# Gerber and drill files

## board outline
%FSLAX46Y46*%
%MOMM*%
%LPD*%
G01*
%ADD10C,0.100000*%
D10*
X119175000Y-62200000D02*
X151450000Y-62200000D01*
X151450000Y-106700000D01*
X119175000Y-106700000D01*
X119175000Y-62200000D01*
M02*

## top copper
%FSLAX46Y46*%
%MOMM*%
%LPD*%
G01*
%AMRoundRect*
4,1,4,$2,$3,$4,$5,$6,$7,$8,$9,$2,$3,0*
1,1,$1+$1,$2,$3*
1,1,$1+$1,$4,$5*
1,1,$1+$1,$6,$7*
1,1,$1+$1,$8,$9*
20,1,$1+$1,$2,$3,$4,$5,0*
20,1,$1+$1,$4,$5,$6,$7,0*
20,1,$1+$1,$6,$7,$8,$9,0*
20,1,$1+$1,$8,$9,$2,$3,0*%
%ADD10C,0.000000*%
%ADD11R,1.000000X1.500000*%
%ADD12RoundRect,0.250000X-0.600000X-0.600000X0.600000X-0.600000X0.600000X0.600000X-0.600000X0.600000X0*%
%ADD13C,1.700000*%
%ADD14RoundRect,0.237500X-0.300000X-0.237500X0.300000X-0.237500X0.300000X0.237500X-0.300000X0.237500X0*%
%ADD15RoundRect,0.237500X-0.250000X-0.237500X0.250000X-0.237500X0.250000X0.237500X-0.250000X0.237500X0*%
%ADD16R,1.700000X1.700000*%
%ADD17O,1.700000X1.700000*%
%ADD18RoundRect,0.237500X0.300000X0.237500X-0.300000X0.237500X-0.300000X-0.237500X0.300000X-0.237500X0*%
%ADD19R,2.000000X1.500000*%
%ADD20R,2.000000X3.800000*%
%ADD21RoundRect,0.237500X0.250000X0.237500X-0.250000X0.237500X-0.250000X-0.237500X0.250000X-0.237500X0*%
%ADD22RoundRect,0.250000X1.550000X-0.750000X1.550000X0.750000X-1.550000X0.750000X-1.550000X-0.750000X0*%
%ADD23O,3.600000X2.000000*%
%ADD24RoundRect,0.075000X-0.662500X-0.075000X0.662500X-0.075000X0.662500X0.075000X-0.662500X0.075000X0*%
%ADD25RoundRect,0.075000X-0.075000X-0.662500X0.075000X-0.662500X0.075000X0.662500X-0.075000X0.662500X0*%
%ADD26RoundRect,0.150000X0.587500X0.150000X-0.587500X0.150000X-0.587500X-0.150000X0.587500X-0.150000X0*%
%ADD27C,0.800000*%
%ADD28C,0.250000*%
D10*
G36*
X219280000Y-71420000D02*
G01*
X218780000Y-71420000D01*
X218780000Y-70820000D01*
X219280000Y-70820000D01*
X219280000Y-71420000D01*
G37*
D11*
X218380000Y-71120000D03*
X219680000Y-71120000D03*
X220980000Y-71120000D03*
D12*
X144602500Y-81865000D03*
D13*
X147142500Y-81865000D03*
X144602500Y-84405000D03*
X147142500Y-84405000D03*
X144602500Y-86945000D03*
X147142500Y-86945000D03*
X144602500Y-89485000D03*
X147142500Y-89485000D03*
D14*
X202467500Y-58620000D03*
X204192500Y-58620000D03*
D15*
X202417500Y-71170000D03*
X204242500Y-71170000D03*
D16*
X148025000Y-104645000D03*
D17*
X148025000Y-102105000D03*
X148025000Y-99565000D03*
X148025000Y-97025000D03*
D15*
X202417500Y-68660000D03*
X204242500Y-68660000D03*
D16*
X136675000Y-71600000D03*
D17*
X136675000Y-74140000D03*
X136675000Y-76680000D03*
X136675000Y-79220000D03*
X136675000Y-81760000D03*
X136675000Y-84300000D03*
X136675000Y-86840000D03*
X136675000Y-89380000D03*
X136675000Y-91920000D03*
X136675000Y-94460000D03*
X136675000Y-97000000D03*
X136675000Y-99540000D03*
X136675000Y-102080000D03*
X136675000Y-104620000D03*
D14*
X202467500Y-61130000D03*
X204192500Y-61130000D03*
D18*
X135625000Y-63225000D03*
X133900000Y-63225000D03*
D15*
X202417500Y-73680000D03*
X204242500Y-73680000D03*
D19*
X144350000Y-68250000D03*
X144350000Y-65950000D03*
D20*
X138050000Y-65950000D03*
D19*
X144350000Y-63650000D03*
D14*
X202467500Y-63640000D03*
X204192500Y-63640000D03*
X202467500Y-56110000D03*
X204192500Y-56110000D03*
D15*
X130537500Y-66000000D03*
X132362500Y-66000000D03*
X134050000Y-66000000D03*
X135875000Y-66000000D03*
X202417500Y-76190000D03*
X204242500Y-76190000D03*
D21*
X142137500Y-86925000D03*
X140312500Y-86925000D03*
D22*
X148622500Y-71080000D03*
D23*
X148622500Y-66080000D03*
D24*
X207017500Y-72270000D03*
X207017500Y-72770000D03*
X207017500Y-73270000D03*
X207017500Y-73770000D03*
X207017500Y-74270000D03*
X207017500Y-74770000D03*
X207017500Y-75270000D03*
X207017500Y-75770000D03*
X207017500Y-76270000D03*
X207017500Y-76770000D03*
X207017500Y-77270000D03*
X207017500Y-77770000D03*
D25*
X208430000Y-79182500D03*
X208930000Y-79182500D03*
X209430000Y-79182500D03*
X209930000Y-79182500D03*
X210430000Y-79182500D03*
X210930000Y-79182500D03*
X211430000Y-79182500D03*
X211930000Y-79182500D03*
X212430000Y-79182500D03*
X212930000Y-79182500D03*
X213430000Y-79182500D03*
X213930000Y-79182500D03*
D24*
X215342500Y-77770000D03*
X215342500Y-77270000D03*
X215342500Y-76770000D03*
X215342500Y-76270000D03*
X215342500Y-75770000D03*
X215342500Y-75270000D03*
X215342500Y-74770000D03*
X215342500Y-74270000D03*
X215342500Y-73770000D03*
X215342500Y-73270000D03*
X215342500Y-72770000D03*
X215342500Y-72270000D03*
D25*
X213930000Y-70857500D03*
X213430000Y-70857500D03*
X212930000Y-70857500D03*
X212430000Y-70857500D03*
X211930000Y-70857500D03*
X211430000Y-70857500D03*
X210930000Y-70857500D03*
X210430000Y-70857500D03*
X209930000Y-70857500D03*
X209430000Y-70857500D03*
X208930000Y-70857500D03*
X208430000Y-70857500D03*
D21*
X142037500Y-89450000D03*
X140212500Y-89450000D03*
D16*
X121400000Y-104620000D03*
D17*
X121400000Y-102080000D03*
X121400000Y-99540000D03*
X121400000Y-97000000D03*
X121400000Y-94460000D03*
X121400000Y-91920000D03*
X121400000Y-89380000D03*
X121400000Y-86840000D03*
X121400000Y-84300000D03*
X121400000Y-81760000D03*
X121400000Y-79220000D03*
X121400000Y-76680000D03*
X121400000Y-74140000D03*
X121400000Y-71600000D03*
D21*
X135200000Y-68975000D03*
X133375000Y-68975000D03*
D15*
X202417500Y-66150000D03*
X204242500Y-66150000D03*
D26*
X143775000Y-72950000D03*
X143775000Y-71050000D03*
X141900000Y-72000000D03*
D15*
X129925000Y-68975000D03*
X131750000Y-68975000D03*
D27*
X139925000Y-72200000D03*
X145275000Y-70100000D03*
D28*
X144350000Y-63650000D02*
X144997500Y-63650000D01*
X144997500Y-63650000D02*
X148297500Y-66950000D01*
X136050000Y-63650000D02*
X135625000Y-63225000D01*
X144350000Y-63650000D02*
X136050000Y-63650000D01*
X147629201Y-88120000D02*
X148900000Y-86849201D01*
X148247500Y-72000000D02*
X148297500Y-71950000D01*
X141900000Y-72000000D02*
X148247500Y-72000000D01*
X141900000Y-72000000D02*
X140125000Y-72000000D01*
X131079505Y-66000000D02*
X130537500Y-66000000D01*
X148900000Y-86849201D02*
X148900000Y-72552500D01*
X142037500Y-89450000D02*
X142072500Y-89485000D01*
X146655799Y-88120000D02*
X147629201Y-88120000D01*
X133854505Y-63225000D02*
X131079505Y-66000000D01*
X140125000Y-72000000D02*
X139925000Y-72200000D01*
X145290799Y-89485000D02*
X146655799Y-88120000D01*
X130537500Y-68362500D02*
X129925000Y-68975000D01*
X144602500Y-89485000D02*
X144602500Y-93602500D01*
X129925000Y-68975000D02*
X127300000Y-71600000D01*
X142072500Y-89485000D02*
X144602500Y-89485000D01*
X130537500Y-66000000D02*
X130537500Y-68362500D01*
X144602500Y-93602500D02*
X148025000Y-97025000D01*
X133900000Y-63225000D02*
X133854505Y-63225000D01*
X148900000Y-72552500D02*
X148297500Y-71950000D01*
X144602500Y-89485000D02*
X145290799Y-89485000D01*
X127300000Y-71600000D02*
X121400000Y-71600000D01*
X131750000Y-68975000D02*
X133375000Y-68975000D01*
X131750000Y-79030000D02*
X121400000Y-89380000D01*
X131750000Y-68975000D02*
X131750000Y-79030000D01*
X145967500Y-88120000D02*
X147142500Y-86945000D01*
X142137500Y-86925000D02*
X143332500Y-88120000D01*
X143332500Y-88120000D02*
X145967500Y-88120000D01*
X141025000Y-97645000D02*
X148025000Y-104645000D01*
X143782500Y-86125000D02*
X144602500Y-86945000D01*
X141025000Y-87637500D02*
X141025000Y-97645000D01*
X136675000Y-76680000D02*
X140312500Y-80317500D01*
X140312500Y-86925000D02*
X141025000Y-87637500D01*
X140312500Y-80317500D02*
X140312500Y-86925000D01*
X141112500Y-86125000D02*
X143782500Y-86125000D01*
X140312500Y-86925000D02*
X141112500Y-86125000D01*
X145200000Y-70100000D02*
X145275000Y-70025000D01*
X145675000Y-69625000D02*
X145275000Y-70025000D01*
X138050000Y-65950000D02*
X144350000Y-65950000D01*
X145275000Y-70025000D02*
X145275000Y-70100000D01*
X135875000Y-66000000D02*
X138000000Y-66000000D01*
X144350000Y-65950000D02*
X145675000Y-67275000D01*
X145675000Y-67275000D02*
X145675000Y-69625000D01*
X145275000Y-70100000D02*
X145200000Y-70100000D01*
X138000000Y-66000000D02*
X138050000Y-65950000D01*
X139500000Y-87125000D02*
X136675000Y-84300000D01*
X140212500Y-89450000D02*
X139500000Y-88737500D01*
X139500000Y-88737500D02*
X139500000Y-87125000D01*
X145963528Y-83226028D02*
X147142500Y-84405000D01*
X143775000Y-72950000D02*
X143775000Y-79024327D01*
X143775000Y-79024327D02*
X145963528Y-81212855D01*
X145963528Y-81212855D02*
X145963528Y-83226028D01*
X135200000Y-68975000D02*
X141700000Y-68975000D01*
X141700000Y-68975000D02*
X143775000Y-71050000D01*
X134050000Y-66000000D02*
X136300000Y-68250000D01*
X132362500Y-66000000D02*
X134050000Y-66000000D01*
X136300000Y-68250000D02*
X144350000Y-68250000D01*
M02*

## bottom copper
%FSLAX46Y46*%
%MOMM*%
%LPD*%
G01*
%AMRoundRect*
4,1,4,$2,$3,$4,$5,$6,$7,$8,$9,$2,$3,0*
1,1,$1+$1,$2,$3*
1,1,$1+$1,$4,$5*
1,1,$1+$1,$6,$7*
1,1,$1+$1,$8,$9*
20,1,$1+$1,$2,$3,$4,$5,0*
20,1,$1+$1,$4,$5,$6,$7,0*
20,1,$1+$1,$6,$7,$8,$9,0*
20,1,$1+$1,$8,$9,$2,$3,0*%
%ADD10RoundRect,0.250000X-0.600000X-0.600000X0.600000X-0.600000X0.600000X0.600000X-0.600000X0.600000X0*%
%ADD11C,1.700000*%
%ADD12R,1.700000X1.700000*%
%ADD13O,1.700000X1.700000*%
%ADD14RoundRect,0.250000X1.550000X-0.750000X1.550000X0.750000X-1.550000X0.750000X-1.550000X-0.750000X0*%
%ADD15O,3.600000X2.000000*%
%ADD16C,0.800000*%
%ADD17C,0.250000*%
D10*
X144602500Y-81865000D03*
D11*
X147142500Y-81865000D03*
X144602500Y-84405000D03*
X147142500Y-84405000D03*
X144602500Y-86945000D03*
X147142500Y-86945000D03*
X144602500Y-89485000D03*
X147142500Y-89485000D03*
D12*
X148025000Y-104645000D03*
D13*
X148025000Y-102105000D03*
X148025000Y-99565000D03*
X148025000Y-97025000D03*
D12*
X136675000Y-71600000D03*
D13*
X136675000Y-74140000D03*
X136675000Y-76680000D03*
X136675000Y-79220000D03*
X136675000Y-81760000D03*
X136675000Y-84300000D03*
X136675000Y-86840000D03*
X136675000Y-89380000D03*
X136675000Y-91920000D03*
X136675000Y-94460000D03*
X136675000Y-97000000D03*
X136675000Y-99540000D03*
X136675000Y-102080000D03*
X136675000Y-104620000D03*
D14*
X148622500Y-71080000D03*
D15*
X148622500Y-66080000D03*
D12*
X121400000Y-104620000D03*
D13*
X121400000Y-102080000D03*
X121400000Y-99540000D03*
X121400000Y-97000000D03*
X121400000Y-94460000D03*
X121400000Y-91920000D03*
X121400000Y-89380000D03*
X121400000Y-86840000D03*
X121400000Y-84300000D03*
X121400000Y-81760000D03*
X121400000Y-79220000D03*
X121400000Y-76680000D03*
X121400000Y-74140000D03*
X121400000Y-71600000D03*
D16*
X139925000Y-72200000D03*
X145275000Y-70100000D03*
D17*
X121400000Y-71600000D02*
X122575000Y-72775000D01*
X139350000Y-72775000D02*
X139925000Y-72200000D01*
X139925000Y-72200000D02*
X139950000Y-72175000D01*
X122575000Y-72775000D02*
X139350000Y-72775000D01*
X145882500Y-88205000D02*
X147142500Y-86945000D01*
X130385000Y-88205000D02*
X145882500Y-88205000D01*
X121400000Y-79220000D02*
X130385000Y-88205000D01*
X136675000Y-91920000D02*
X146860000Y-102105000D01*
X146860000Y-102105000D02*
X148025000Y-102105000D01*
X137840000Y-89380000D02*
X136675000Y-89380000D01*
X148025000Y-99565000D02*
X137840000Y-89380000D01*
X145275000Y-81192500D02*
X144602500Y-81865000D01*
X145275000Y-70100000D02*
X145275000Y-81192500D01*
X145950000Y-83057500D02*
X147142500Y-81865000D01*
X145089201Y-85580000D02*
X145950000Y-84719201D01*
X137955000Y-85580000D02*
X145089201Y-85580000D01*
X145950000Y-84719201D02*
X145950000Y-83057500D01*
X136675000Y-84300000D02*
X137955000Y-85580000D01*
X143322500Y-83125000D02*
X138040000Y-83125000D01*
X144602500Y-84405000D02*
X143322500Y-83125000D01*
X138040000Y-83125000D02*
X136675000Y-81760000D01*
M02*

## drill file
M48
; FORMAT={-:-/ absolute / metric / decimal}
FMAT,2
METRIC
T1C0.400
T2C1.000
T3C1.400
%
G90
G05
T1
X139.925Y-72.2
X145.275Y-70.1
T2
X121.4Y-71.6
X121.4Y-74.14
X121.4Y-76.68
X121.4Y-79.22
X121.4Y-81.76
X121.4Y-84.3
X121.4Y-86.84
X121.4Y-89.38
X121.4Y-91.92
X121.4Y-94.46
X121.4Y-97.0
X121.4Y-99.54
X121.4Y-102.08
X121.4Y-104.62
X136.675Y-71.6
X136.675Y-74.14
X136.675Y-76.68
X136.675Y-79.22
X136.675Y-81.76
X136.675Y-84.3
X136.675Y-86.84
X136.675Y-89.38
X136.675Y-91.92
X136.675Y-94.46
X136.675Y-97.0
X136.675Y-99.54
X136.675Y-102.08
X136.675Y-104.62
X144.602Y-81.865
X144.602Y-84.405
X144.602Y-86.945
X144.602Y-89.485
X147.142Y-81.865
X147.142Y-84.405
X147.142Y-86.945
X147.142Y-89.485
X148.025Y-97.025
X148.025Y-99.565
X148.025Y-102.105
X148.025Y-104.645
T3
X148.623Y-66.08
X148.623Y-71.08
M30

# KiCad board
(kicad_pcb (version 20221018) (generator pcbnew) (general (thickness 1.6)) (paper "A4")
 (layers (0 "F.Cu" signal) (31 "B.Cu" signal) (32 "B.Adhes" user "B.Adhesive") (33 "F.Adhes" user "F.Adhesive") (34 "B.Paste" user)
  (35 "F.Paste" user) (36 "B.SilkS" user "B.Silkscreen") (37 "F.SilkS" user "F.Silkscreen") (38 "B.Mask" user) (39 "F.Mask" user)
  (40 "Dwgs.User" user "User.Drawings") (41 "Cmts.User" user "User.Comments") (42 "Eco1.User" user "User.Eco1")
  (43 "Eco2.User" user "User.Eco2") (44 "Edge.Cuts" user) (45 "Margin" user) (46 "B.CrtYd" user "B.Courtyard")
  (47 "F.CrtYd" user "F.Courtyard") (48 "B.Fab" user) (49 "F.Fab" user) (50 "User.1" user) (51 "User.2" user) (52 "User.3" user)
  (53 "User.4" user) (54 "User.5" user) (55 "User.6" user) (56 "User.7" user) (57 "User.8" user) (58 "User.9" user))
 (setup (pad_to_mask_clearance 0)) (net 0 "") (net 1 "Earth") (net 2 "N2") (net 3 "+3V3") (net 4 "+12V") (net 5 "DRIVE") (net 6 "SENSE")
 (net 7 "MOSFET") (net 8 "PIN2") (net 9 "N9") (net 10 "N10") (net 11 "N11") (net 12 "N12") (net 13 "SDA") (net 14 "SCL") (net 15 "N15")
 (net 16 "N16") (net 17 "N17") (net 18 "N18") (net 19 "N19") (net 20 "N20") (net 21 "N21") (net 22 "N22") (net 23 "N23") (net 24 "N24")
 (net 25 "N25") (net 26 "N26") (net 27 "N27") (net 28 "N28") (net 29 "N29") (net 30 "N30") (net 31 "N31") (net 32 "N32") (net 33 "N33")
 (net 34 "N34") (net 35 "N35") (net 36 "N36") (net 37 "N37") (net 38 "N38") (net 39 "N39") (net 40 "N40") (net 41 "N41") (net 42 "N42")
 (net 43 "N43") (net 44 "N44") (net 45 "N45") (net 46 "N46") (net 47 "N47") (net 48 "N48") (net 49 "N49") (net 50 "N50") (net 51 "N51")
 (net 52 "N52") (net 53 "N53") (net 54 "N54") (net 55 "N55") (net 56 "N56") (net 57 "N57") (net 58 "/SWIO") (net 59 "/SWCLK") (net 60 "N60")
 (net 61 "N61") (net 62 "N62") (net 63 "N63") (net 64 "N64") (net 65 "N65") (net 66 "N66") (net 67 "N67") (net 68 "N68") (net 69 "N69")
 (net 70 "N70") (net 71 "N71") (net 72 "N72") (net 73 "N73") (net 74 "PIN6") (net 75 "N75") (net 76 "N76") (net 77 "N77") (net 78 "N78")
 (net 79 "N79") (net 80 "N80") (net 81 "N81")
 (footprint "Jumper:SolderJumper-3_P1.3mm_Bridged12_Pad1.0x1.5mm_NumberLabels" (layer "F.Cu") (at 219.68 71.12)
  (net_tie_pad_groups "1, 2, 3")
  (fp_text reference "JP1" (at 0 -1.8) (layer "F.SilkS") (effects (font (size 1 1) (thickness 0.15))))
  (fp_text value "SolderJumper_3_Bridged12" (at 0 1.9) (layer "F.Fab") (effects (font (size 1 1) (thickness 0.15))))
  (fp_poly (pts (xy -0.9 -0.3) (xy -0.4 -0.3) (xy -0.4 0.3) (xy -0.9 0.3)) (stroke (width 0) (type solid)) (fill solid) (layer "F.Cu"))
  (pad "1" smd rect (at -1.3 0) (size 1 1.5) (layers "F.Cu" "F.Mask") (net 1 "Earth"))
  (pad "2" smd rect (at 0 0) (size 1 1.5) (layers "F.Cu" "F.Mask") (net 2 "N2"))
  (pad "3" smd rect (at 1.3 0) (size 1 1.5) (layers "F.Cu" "F.Mask") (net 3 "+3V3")))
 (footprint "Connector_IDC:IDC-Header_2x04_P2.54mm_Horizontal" (layer "F.Cu") (at 144.6025 81.865)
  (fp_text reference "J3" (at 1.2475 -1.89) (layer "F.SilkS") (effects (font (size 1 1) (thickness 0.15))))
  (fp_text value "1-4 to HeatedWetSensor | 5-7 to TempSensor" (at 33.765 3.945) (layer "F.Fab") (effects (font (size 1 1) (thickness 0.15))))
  (pad "1" thru_hole roundrect (at 0 0) (size 1.7 1.7) (drill 1) (layers "*.Cu" "*.Mask") (roundrect_rratio 0.147059) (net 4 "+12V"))
  (pad "2" thru_hole circle (at 2.54 0) (size 1.7 1.7) (drill 1) (layers "*.Cu" "*.Mask") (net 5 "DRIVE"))
  (pad "3" thru_hole circle (at 0 2.54) (size 1.7 1.7) (drill 1) (layers "*.Cu" "*.Mask") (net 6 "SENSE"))
  (pad "4" thru_hole circle (at 2.54 2.54) (size 1.7 1.7) (drill 1) (layers "*.Cu" "*.Mask") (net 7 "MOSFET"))
  (pad "5" thru_hole circle (at 0 5.08) (size 1.7 1.7) (drill 1) (layers "*.Cu" "*.Mask") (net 3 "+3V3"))
  (pad "6" thru_hole circle (at 2.54 5.08) (size 1.7 1.7) (drill 1) (layers "*.Cu" "*.Mask") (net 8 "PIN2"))
  (pad "7" thru_hole circle (at 0 7.62) (size 1.7 1.7) (drill 1) (layers "*.Cu" "*.Mask") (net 1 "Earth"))
  (pad "8" thru_hole circle (at 2.54 7.62) (size 1.7 1.7) (drill 1) (layers "*.Cu" "*.Mask") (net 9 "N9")))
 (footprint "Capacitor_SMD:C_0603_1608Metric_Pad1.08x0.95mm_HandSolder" (layer "F.Cu") (at 203.33 58.62)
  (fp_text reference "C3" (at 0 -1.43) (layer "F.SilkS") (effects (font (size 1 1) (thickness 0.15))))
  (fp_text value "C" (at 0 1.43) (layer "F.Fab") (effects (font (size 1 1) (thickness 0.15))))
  (pad "1" smd roundrect (at -0.8625 0) (size 1.075 0.95) (layers "F.Cu" "F.Paste" "F.Mask") (roundrect_rratio 0.25) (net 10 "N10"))
  (pad "2" smd roundrect (at 0.8625 0) (size 1.075 0.95) (layers "F.Cu" "F.Paste" "F.Mask") (roundrect_rratio 0.25) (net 1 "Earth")))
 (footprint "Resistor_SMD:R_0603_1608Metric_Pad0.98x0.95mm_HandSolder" (layer "F.Cu") (at 203.33 71.17)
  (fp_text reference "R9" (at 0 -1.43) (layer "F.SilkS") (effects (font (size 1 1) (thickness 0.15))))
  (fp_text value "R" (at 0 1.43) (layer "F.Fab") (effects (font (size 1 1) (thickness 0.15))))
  (pad "1" smd roundrect (at -0.9125 0) (size 0.975 0.95) (layers "F.Cu" "F.Paste" "F.Mask") (roundrect_rratio 0.25) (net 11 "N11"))
  (pad "2" smd roundrect (at 0.9125 0) (size 0.975 0.95) (layers "F.Cu" "F.Paste" "F.Mask") (roundrect_rratio 0.25) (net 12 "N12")))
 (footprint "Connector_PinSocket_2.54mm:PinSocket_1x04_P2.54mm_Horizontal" (layer "F.Cu") (at 148.025 104.645 180)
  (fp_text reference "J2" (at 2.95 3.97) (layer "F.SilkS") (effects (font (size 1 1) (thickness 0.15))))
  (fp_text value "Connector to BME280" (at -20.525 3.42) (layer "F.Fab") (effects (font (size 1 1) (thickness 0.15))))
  (pad "1" thru_hole rect (at 0 0 180) (size 1.7 1.7) (drill 1) (layers "*.Cu" "*.Mask") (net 3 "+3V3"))
  (pad "2" thru_hole oval (at 0 2.54 180) (size 1.7 1.7) (drill 1) (layers "*.Cu" "*.Mask") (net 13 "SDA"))
  (pad "3" thru_hole oval (at 0 5.08 180) (size 1.7 1.7) (drill 1) (layers "*.Cu" "*.Mask") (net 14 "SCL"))
  (pad "4" thru_hole oval (at 0 7.62 180) (size 1.7 1.7) (drill 1) (layers "*.Cu" "*.Mask") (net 1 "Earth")))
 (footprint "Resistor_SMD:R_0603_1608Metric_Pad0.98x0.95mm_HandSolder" (layer "F.Cu") (at 203.33 68.66)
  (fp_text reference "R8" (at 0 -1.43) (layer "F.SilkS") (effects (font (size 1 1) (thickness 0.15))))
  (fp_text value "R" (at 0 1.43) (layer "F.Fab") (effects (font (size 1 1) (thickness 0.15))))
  (pad "1" smd roundrect (at -0.9125 0) (size 0.975 0.95) (layers "F.Cu" "F.Paste" "F.Mask") (roundrect_rratio 0.25) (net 11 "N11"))
  (pad "2" smd roundrect (at 0.9125 0) (size 0.975 0.95) (layers "F.Cu" "F.Paste" "F.Mask") (roundrect_rratio 0.25) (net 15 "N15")))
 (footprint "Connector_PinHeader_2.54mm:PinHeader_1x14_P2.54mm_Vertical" (layer "F.Cu") (at 136.675 71.6)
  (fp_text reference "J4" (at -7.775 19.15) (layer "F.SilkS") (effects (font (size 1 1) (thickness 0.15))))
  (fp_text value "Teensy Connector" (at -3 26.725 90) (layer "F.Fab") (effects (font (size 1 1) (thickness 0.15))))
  (pad "1" thru_hole rect (at 0 0) (size 1.7 1.7) (drill 1) (layers "*.Cu" "*.Mask") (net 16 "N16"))
  (pad "2" thru_hole oval (at 0 2.54) (size 1.7 1.7) (drill 1) (layers "*.Cu" "*.Mask") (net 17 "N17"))
  (pad "3" thru_hole oval (at 0 5.08) (size 1.7 1.7) (drill 1) (layers "*.Cu" "*.Mask") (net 3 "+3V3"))
  (pad "4" thru_hole oval (at 0 7.62) (size 1.7 1.7) (drill 1) (layers "*.Cu" "*.Mask") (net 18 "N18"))
  (pad "5" thru_hole oval (at 0 10.16) (size 1.7 1.7) (drill 1) (layers "*.Cu" "*.Mask") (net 6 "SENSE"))
  (pad "6" thru_hole oval (at 0 12.7) (size 1.7 1.7) (drill 1) (layers "*.Cu" "*.Mask") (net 5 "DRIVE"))
  (pad "7" thru_hole oval (at 0 15.24) (size 1.7 1.7) (drill 1) (layers "*.Cu" "*.Mask") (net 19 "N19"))
  (pad "8" thru_hole oval (at 0 17.78) (size 1.7 1.7) (drill 1) (layers "*.Cu" "*.Mask") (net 14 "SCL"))
  (pad "9" thru_hole oval (at 0 20.32) (size 1.7 1.7) (drill 1) (layers "*.Cu" "*.Mask") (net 13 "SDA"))
  (pad "10" thru_hole oval (at 0 22.86) (size 1.7 1.7) (drill 1) (layers "*.Cu" "*.Mask") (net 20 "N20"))
  (pad "11" thru_hole oval (at 0 25.4) (size 1.7 1.7) (drill 1) (layers "*.Cu" "*.Mask") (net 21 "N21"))
  (pad "12" thru_hole oval (at 0 27.94) (size 1.7 1.7) (drill 1) (layers "*.Cu" "*.Mask") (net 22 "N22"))
  (pad "13" thru_hole oval (at 0 30.48) (size 1.7 1.7) (drill 1) (layers "*.Cu" "*.Mask") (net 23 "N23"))
  (pad "14" thru_hole oval (at 0 33.02) (size 1.7 1.7) (drill 1) (layers "*.Cu" "*.Mask") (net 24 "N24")))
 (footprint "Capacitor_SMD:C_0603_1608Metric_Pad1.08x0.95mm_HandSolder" (layer "F.Cu") (at 203.33 61.13)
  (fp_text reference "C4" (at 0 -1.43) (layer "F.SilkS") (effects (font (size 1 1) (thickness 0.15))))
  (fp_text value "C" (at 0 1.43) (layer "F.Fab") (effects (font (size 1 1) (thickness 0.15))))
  (pad "1" smd roundrect (at -0.8625 0) (size 1.075 0.95) (layers "F.Cu" "F.Paste" "F.Mask") (roundrect_rratio 0.25) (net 4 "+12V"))
  (pad "2" smd roundrect (at 0.8625 0) (size 1.075 0.95) (layers "F.Cu" "F.Paste" "F.Mask") (roundrect_rratio 0.25) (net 1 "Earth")))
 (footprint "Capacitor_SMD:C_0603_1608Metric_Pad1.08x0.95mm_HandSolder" (layer "F.Cu") (at 134.7625 63.225 180)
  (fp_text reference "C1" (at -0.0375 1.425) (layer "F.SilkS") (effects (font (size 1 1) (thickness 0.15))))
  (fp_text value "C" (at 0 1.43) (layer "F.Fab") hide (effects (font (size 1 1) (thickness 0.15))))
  (pad "1" smd roundrect (at -0.8625 0 180) (size 1.075 0.95) (layers "F.Cu" "F.Paste" "F.Mask") (roundrect_rratio 0.25) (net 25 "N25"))
  (pad "2" smd roundrect (at 0.8625 0 180) (size 1.075 0.95) (layers "F.Cu" "F.Paste" "F.Mask") (roundrect_rratio 0.25) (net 1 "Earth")))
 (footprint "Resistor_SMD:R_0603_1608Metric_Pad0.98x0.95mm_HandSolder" (layer "F.Cu") (at 203.33 73.68)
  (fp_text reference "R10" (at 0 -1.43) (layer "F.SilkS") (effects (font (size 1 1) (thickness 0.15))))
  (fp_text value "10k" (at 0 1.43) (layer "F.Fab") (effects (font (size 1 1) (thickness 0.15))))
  (pad "1" smd roundrect (at -0.9125 0) (size 0.975 0.95) (layers "F.Cu" "F.Paste" "F.Mask") (roundrect_rratio 0.25) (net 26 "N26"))
  (pad "2" smd roundrect (at 0.9125 0) (size 0.975 0.95) (layers "F.Cu" "F.Paste" "F.Mask") (roundrect_rratio 0.25) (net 3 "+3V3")))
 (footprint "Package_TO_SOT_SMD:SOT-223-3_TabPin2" (layer "F.Cu") (at 141.2 65.95 180)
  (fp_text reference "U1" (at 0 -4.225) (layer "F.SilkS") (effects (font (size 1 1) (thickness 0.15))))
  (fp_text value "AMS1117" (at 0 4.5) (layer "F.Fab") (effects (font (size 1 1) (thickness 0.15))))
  (pad "1" smd rect (at -3.15 -2.3 180) (size 2 1.5) (layers "F.Cu" "F.Paste" "F.Mask") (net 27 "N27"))
  (pad "2" smd rect (at -3.15 0 180) (size 2 1.5) (layers "F.Cu" "F.Paste" "F.Mask") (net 4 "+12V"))
  (pad "2" smd rect (at 3.15 0 180) (size 2 3.8) (layers "F.Cu" "F.Paste" "F.Mask") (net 4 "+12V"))
  (pad "3" smd rect (at -3.15 2.3 180) (size 2 1.5) (layers "F.Cu" "F.Paste" "F.Mask") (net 25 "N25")))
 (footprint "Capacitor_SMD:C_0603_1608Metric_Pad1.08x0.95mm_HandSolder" (layer "F.Cu") (at 203.33 63.64)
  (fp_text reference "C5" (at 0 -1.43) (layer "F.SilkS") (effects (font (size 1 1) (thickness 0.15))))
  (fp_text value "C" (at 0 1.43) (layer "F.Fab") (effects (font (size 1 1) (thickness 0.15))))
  (pad "1" smd roundrect (at -0.8625 0) (size 1.075 0.95) (layers "F.Cu" "F.Paste" "F.Mask") (roundrect_rratio 0.25) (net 26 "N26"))
  (pad "2" smd roundrect (at 0.8625 0) (size 1.075 0.95) (layers "F.Cu" "F.Paste" "F.Mask") (roundrect_rratio 0.25) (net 1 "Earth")))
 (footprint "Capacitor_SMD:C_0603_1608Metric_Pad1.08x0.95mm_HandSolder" (layer "F.Cu") (at 203.33 56.11)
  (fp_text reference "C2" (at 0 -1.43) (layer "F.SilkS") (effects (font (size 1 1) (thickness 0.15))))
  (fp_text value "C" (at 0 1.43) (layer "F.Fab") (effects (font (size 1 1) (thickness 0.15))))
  (pad "1" smd roundrect (at -0.8625 0) (size 1.075 0.95) (layers "F.Cu" "F.Paste" "F.Mask") (roundrect_rratio 0.25) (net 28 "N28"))
  (pad "2" smd roundrect (at 0.8625 0) (size 1.075 0.95) (layers "F.Cu" "F.Paste" "F.Mask") (roundrect_rratio 0.25) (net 1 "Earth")))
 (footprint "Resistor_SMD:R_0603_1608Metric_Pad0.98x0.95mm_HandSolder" (layer "F.Cu") (at 131.45 66)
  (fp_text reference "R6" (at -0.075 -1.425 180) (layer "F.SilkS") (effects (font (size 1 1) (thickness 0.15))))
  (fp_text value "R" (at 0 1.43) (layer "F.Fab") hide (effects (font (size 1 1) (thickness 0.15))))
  (pad "1" smd roundrect (at -0.9125 0) (size 0.975 0.95) (layers "F.Cu" "F.Paste" "F.Mask") (roundrect_rratio 0.25) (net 1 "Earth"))
  (pad "2" smd roundrect (at 0.9125 0) (size 0.975 0.95) (layers "F.Cu" "F.Paste" "F.Mask") (roundrect_rratio 0.25) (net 27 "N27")))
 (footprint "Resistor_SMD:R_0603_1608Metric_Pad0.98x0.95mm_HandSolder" (layer "F.Cu") (at 134.9625 66)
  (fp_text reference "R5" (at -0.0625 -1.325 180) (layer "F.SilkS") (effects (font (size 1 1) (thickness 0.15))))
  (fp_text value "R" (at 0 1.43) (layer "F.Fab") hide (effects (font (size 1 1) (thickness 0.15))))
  (pad "1" smd roundrect (at -0.9125 0) (size 0.975 0.95) (layers "F.Cu" "F.Paste" "F.Mask") (roundrect_rratio 0.25) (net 27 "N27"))
  (pad "2" smd roundrect (at 0.9125 0) (size 0.975 0.95) (layers "F.Cu" "F.Paste" "F.Mask") (roundrect_rratio 0.25) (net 4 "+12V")))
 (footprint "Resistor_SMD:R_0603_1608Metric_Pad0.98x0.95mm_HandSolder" (layer "F.Cu") (at 203.33 76.19)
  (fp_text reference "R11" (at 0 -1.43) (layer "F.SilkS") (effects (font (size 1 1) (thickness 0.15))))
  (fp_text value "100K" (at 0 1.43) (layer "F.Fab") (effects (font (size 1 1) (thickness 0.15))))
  (pad "1" smd roundrect (at -0.9125 0) (size 0.975 0.95) (layers "F.Cu" "F.Paste" "F.Mask") (roundrect_rratio 0.25) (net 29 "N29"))
  (pad "2" smd roundrect (at 0.9125 0) (size 0.975 0.95) (layers "F.Cu" "F.Paste" "F.Mask") (roundrect_rratio 0.25) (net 2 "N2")))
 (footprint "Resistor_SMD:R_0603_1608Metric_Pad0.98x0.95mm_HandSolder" (layer "F.Cu") (at 141.225 86.925 180)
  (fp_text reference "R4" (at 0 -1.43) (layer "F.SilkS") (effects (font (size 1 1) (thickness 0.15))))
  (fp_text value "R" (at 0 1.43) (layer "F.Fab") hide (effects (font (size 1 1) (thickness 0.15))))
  (pad "1" smd roundrect (at -0.9125 0 180) (size 0.975 0.95) (layers "F.Cu" "F.Paste" "F.Mask") (roundrect_rratio 0.25) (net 8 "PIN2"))
  (pad "2" smd roundrect (at 0.9125 0 180) (size 0.975 0.95) (layers "F.Cu" "F.Paste" "F.Mask") (roundrect_rratio 0.25) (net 3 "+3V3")))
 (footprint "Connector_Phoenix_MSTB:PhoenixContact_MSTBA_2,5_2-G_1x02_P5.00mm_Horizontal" (layer "F.Cu") (at 148.6225 71.08 90)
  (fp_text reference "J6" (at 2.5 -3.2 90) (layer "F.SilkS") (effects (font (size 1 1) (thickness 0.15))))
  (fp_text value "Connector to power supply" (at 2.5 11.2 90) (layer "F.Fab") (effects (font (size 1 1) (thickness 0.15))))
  (pad "1" thru_hole roundrect (at 0 0 90) (size 2 3.6) (drill 1.4) (layers "*.Cu" "*.Mask") (roundrect_rratio 0.125) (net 1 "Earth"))
  (pad "2" thru_hole oval (at 5 0 90) (size 2 3.6) (drill 1.4) (layers "*.Cu" "*.Mask") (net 10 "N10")))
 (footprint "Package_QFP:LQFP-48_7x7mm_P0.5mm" (layer "F.Cu") (at 211.18 75.02)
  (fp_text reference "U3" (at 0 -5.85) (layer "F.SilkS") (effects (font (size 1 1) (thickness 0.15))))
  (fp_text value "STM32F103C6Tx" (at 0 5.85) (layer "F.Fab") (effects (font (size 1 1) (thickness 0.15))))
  (pad "1" smd roundrect (at -4.1625 -2.75) (size 1.475 0.3) (layers "F.Cu" "F.Paste" "F.Mask") (roundrect_rratio 0.25) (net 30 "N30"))
  (pad "2" smd roundrect (at -4.1625 -2.25) (size 1.475 0.3) (layers "F.Cu" "F.Paste" "F.Mask") (roundrect_rratio 0.25) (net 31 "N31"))
  (pad "3" smd roundrect (at -4.1625 -1.75) (size 1.475 0.3) (layers "F.Cu" "F.Paste" "F.Mask") (roundrect_rratio 0.25) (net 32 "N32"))
  (pad "4" smd roundrect (at -4.1625 -1.25) (size 1.475 0.3) (layers "F.Cu" "F.Paste" "F.Mask") (roundrect_rratio 0.25) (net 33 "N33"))
  (pad "5" smd roundrect (at -4.1625 -0.75) (size 1.475 0.3) (layers "F.Cu" "F.Paste" "F.Mask") (roundrect_rratio 0.25) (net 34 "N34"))
  (pad "6" smd roundrect (at -4.1625 -0.25) (size 1.475 0.3) (layers "F.Cu" "F.Paste" "F.Mask") (roundrect_rratio 0.25) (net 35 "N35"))
  (pad "7" smd roundrect (at -4.1625 0.25) (size 1.475 0.3) (layers "F.Cu" "F.Paste" "F.Mask") (roundrect_rratio 0.25) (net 26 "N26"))
  (pad "8" smd roundrect (at -4.1625 0.75) (size 1.475 0.3) (layers "F.Cu" "F.Paste" "F.Mask") (roundrect_rratio 0.25) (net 1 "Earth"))
  (pad "9" smd roundrect (at -4.1625 1.25) (size 1.475 0.3) (layers "F.Cu" "F.Paste" "F.Mask") (roundrect_rratio 0.25) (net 3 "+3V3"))
  (pad "10" smd roundrect (at -4.1625 1.75) (size 1.475 0.3) (layers "F.Cu" "F.Paste" "F.Mask") (roundrect_rratio 0.25) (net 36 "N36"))
  (pad "11" smd roundrect (at -4.1625 2.25) (size 1.475 0.3) (layers "F.Cu" "F.Paste" "F.Mask") (roundrect_rratio 0.25) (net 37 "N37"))
  (pad "12" smd roundrect (at -4.1625 2.75) (size 1.475 0.3) (layers "F.Cu" "F.Paste" "F.Mask") (roundrect_rratio 0.25) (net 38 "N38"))
  (pad "13" smd roundrect (at -2.75 4.1625) (size 0.3 1.475) (layers "F.Cu" "F.Paste" "F.Mask") (roundrect_rratio 0.25) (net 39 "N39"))
  (pad "14" smd roundrect (at -2.25 4.1625) (size 0.3 1.475) (layers "F.Cu" "F.Paste" "F.Mask") (roundrect_rratio 0.25) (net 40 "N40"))
  (pad "15" smd roundrect (at -1.75 4.1625) (size 0.3 1.475) (layers "F.Cu" "F.Paste" "F.Mask") (roundrect_rratio 0.25) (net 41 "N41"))
  (pad "16" smd roundrect (at -1.25 4.1625) (size 0.3 1.475) (layers "F.Cu" "F.Paste" "F.Mask") (roundrect_rratio 0.25) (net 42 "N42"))
  (pad "17" smd roundrect (at -0.75 4.1625) (size 0.3 1.475) (layers "F.Cu" "F.Paste" "F.Mask") (roundrect_rratio 0.25) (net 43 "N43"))
  (pad "18" smd roundrect (at -0.25 4.1625) (size 0.3 1.475) (layers "F.Cu" "F.Paste" "F.Mask") (roundrect_rratio 0.25) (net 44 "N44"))
  (pad "19" smd roundrect (at 0.25 4.1625) (size 0.3 1.475) (layers "F.Cu" "F.Paste" "F.Mask") (roundrect_rratio 0.25) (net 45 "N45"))
  (pad "20" smd roundrect (at 0.75 4.1625) (size 0.3 1.475) (layers "F.Cu" "F.Paste" "F.Mask") (roundrect_rratio 0.25) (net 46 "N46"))
  (pad "21" smd roundrect (at 1.25 4.1625) (size 0.3 1.475) (layers "F.Cu" "F.Paste" "F.Mask") (roundrect_rratio 0.25) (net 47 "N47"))
  (pad "22" smd roundrect (at 1.75 4.1625) (size 0.3 1.475) (layers "F.Cu" "F.Paste" "F.Mask") (roundrect_rratio 0.25) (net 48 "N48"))
  (pad "23" smd roundrect (at 2.25 4.1625) (size 0.3 1.475) (layers "F.Cu" "F.Paste" "F.Mask") (roundrect_rratio 0.25) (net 1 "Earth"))
  (pad "24" smd roundrect (at 2.75 4.1625) (size 0.3 1.475) (layers "F.Cu" "F.Paste" "F.Mask") (roundrect_rratio 0.25) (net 3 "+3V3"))
  (pad "25" smd roundrect (at 4.1625 2.75) (size 1.475 0.3) (layers "F.Cu" "F.Paste" "F.Mask") (roundrect_rratio 0.25) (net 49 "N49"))
  (pad "26" smd roundrect (at 4.1625 2.25) (size 1.475 0.3) (layers "F.Cu" "F.Paste" "F.Mask") (roundrect_rratio 0.25) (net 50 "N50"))
  (pad "27" smd roundrect (at 4.1625 1.75) (size 1.475 0.3) (layers "F.Cu" "F.Paste" "F.Mask") (roundrect_rratio 0.25) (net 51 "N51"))
  (pad "28" smd roundrect (at 4.1625 1.25) (size 1.475 0.3) (layers "F.Cu" "F.Paste" "F.Mask") (roundrect_rratio 0.25) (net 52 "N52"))
  (pad "29" smd roundrect (at 4.1625 0.75) (size 1.475 0.3) (layers "F.Cu" "F.Paste" "F.Mask") (roundrect_rratio 0.25) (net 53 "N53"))
  (pad "30" smd roundrect (at 4.1625 0.25) (size 1.475 0.3) (layers "F.Cu" "F.Paste" "F.Mask") (roundrect_rratio 0.25) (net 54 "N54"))
  (pad "31" smd roundrect (at 4.1625 -0.25) (size 1.475 0.3) (layers "F.Cu" "F.Paste" "F.Mask") (roundrect_rratio 0.25) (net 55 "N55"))
  (pad "32" smd roundrect (at 4.1625 -0.75) (size 1.475 0.3) (layers "F.Cu" "F.Paste" "F.Mask") (roundrect_rratio 0.25) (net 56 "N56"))
  (pad "33" smd roundrect (at 4.1625 -1.25) (size 1.475 0.3) (layers "F.Cu" "F.Paste" "F.Mask") (roundrect_rratio 0.25) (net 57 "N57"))
  (pad "34" smd roundrect (at 4.1625 -1.75) (size 1.475 0.3) (layers "F.Cu" "F.Paste" "F.Mask") (roundrect_rratio 0.25) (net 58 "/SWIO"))
  (pad "35" smd roundrect (at 4.1625 -2.25) (size 1.475 0.3) (layers "F.Cu" "F.Paste" "F.Mask") (roundrect_rratio 0.25) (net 1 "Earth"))
  (pad "36" smd roundrect (at 4.1625 -2.75) (size 1.475 0.3) (layers "F.Cu" "F.Paste" "F.Mask") (roundrect_rratio 0.25) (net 3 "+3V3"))
  (pad "37" smd roundrect (at 2.75 -4.1625) (size 0.3 1.475) (layers "F.Cu" "F.Paste" "F.Mask") (roundrect_rratio 0.25) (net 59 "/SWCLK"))
  (pad "38" smd roundrect (at 2.25 -4.1625) (size 0.3 1.475) (layers "F.Cu" "F.Paste" "F.Mask") (roundrect_rratio 0.25) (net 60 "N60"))
  (pad "39" smd roundrect (at 1.75 -4.1625) (size 0.3 1.475) (layers "F.Cu" "F.Paste" "F.Mask") (roundrect_rratio 0.25) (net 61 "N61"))
  (pad "40" smd roundrect (at 1.25 -4.1625) (size 0.3 1.475) (layers "F.Cu" "F.Paste" "F.Mask") (roundrect_rratio 0.25) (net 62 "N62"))
  (pad "41" smd roundrect (at 0.75 -4.1625) (size 0.3 1.475) (layers "F.Cu" "F.Paste" "F.Mask") (roundrect_rratio 0.25) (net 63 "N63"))
  (pad "42" smd roundrect (at 0.25 -4.1625) (size 0.3 1.475) (layers "F.Cu" "F.Paste" "F.Mask") (roundrect_rratio 0.25) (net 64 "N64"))
  (pad "43" smd roundrect (at -0.25 -4.1625) (size 0.3 1.475) (layers "F.Cu" "F.Paste" "F.Mask") (roundrect_rratio 0.25) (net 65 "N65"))
  (pad "44" smd roundrect (at -0.75 -4.1625) (size 0.3 1.475) (layers "F.Cu" "F.Paste" "F.Mask") (roundrect_rratio 0.25) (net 29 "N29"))
  (pad "45" smd roundrect (at -1.25 -4.1625) (size 0.3 1.475) (layers "F.Cu" "F.Paste" "F.Mask") (roundrect_rratio 0.25) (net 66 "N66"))
  (pad "46" smd roundrect (at -1.75 -4.1625) (size 0.3 1.475) (layers "F.Cu" "F.Paste" "F.Mask") (roundrect_rratio 0.25) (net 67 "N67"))
  (pad "47" smd roundrect (at -2.25 -4.1625) (size 0.3 1.475) (layers "F.Cu" "F.Paste" "F.Mask") (roundrect_rratio 0.25) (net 1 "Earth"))
  (pad "48" smd roundrect (at -2.75 -4.1625) (size 0.3 1.475) (layers "F.Cu" "F.Paste" "F.Mask") (roundrect_rratio 0.25) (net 3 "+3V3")))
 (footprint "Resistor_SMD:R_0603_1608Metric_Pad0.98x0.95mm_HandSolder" (layer "F.Cu") (at 141.125 89.45 180)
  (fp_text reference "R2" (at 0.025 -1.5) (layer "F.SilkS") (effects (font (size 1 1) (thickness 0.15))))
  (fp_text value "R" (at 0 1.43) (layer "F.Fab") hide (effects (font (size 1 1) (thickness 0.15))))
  (pad "1" smd roundrect (at -0.9125 0 180) (size 0.975 0.95) (layers "F.Cu" "F.Paste" "F.Mask") (roundrect_rratio 0.25) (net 1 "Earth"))
  (pad "2" smd roundrect (at 0.9125 0 180) (size 0.975 0.95) (layers "F.Cu" "F.Paste" "F.Mask") (roundrect_rratio 0.25) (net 5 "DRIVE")))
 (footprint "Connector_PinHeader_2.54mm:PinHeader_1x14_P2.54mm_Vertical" (layer "F.Cu") (at 121.4 104.62 180)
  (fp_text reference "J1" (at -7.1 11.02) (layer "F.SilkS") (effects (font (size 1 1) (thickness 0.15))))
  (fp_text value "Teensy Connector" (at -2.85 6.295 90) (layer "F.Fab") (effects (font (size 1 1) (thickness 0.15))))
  (pad "1" thru_hole rect (at 0 0 180) (size 1.7 1.7) (drill 1) (layers "*.Cu" "*.Mask") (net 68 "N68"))
  (pad "2" thru_hole oval (at 0 2.54 180) (size 1.7 1.7) (drill 1) (layers "*.Cu" "*.Mask") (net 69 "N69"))
  (pad "3" thru_hole oval (at 0 5.08 180) (size 1.7 1.7) (drill 1) (layers "*.Cu" "*.Mask") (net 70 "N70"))
  (pad "4" thru_hole oval (at 0 7.62 180) (size 1.7 1.7) (drill 1) (layers "*.Cu" "*.Mask") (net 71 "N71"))
  (pad "5" thru_hole oval (at 0 10.16 180) (size 1.7 1.7) (drill 1) (layers "*.Cu" "*.Mask") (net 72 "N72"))
  (pad "6" thru_hole oval (at 0 12.7 180) (size 1.7 1.7) (drill 1) (layers "*.Cu" "*.Mask") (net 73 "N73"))
  (pad "7" thru_hole oval (at 0 15.24 180) (size 1.7 1.7) (drill 1) (layers "*.Cu" "*.Mask") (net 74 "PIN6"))
  (pad "8" thru_hole oval (at 0 17.78 180) (size 1.7 1.7) (drill 1) (layers "*.Cu" "*.Mask") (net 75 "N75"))
  (pad "9" thru_hole oval (at 0 20.32 180) (size 1.7 1.7) (drill 1) (layers "*.Cu" "*.Mask") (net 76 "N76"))
  (pad "10" thru_hole oval (at 0 22.86 180) (size 1.7 1.7) (drill 1) (layers "*.Cu" "*.Mask") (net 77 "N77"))
  (pad "11" thru_hole oval (at 0 25.4 180) (size 1.7 1.7) (drill 1) (layers "*.Cu" "*.Mask") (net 8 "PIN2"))
  (pad "12" thru_hole oval (at 0 27.94 180) (size 1.7 1.7) (drill 1) (layers "*.Cu" "*.Mask") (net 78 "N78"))
  (pad "13" thru_hole oval (at 0 30.48 180) (size 1.7 1.7) (drill 1) (layers "*.Cu" "*.Mask") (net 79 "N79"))
  (pad "14" thru_hole oval (at 0 33.02 180) (size 1.7 1.7) (drill 1) (layers "*.Cu" "*.Mask") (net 1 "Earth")))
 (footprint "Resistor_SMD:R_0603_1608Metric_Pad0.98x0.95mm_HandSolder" (layer "F.Cu") (at 134.2875 68.975 180)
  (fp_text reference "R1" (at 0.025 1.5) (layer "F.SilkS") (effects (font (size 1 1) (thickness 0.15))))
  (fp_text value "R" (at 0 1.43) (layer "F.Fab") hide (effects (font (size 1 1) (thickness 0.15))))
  (pad "1" smd roundrect (at -0.9125 0 180) (size 0.975 0.95) (layers "F.Cu" "F.Paste" "F.Mask") (roundrect_rratio 0.25) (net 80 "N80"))
  (pad "2" smd roundrect (at 0.9125 0 180) (size 0.975 0.95) (layers "F.Cu" "F.Paste" "F.Mask") (roundrect_rratio 0.25) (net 74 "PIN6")))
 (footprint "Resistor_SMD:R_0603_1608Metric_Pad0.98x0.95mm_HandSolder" (layer "F.Cu") (at 203.33 66.15)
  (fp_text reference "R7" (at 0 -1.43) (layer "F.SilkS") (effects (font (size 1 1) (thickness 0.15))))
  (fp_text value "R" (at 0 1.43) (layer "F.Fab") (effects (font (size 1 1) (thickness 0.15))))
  (pad "1" smd roundrect (at -0.9125 0) (size 0.975 0.95) (layers "F.Cu" "F.Paste" "F.Mask") (roundrect_rratio 0.25) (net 1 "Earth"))
  (pad "2" smd roundrect (at 0.9125 0) (size 0.975 0.95) (layers "F.Cu" "F.Paste" "F.Mask") (roundrect_rratio 0.25) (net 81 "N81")))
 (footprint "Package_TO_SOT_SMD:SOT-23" (layer "F.Cu") (at 142.8375 72 180)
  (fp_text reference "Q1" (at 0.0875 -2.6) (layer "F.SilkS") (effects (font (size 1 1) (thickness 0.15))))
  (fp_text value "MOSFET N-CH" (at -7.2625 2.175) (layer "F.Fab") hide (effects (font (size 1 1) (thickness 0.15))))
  (pad "1" smd roundrect (at -0.9375 -0.95 180) (size 1.475 0.6) (layers "F.Cu" "F.Paste" "F.Mask") (roundrect_rratio 0.25) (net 7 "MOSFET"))
  (pad "2" smd roundrect (at -0.9375 0.95 180) (size 1.475 0.6) (layers "F.Cu" "F.Paste" "F.Mask") (roundrect_rratio 0.25) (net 80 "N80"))
  (pad "3" smd roundrect (at 0.9375 0 180) (size 1.475 0.6) (layers "F.Cu" "F.Paste" "F.Mask") (roundrect_rratio 0.25) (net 1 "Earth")))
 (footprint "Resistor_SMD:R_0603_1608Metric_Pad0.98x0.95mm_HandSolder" (layer "F.Cu") (at 130.8375 68.975)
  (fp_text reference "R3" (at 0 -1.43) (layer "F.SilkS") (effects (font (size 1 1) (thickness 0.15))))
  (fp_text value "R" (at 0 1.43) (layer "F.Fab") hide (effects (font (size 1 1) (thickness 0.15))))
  (pad "1" smd roundrect (at -0.9125 0) (size 0.975 0.95) (layers "F.Cu" "F.Paste" "F.Mask") (roundrect_rratio 0.25) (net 1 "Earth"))
  (pad "2" smd roundrect (at 0.9125 0) (size 0.975 0.95) (layers "F.Cu" "F.Paste" "F.Mask") (roundrect_rratio 0.25) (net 74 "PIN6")))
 (gr_rect (start 119.175 62.2) (end 151.45 106.7) (stroke (width 0.1) (type default)) (fill none) (layer "Edge.Cuts"))
 (segment (start 144.35 63.65) (end 144.9975 63.65) (width 0.25) (layer "F.Cu") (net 25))
 (segment (start 144.9975 63.65) (end 148.2975 66.95) (width 0.25) (layer "F.Cu") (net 25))
 (segment (start 136.05 63.65) (end 135.625 63.225) (width 0.25) (layer "F.Cu") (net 25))
 (segment (start 144.35 63.65) (end 136.05 63.65) (width 0.25) (layer "F.Cu") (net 25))
 (segment (start 147.629201 88.12) (end 148.9 86.849201) (width 0.25) (layer "F.Cu") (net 1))
 (segment (start 148.2475 72) (end 148.2975 71.95) (width 0.25) (layer "F.Cu") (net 1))
 (segment (start 141.9 72) (end 148.2475 72) (width 0.25) (layer "F.Cu") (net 1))
 (segment (start 141.9 72) (end 140.125 72) (width 0.25) (layer "F.Cu") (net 1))
 (segment (start 131.079505 66) (end 130.5375 66) (width 0.25) (layer "F.Cu") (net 1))
 (segment (start 148.9 86.849201) (end 148.9 72.5525) (width 0.25) (layer "F.Cu") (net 1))
 (segment (start 142.0375 89.45) (end 142.0725 89.485) (width 0.25) (layer "F.Cu") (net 1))
 (segment (start 146.655799 88.12) (end 147.629201 88.12) (width 0.25) (layer "F.Cu") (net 1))
 (segment (start 133.854505 63.225) (end 131.079505 66) (width 0.25) (layer "F.Cu") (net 1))
 (segment (start 140.125 72) (end 139.925 72.2) (width 0.25) (layer "F.Cu") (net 1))
 (segment (start 145.290799 89.485) (end 146.655799 88.12) (width 0.25) (layer "F.Cu") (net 1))
 (segment (start 130.5375 68.3625) (end 129.925 68.975) (width 0.25) (layer "F.Cu") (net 1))
 (segment (start 144.6025 89.485) (end 144.6025 93.6025) (width 0.25) (layer "F.Cu") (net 1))
 (segment (start 129.925 68.975) (end 127.3 71.6) (width 0.25) (layer "F.Cu") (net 1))
 (segment (start 142.0725 89.485) (end 144.6025 89.485) (width 0.25) (layer "F.Cu") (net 1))
 (segment (start 130.5375 66) (end 130.5375 68.3625) (width 0.25) (layer "F.Cu") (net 1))
 (segment (start 144.6025 93.6025) (end 148.025 97.025) (width 0.25) (layer "F.Cu") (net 1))
 (segment (start 133.9 63.225) (end 133.854505 63.225) (width 0.25) (layer "F.Cu") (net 1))
 (segment (start 148.9 72.5525) (end 148.2975 71.95) (width 0.25) (layer "F.Cu") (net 1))
 (segment (start 144.6025 89.485) (end 145.290799 89.485) (width 0.25) (layer "F.Cu") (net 1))
 (segment (start 127.3 71.6) (end 121.4 71.6) (width 0.25) (layer "F.Cu") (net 1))
 (via (at 139.925 72.2) (size 0.8) (drill 0.4) (layers "F.Cu" "B.Cu") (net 1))
 (segment (start 121.4 71.6) (end 122.575 72.775) (width 0.25) (layer "B.Cu") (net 1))
 (segment (start 139.35 72.775) (end 139.925 72.2) (width 0.25) (layer "B.Cu") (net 1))
 (segment (start 139.925 72.2) (end 139.95 72.175) (width 0.25) (layer "B.Cu") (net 1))
 (segment (start 122.575 72.775) (end 139.35 72.775) (width 0.25) (layer "B.Cu") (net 1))
 (segment (start 131.75 68.975) (end 133.375 68.975) (width 0.25) (layer "F.Cu") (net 74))
 (segment (start 131.75 79.03) (end 121.4 89.38) (width 0.25) (layer "F.Cu") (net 74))
 (segment (start 131.75 68.975) (end 131.75 79.03) (width 0.25) (layer "F.Cu") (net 74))
 (segment (start 145.9675 88.12) (end 147.1425 86.945) (width 0.25) (layer "F.Cu") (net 8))
 (segment (start 142.1375 86.925) (end 143.3325 88.12) (width 0.25) (layer "F.Cu") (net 8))
 (segment (start 143.3325 88.12) (end 145.9675 88.12) (width 0.25) (layer "F.Cu") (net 8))
 (segment (start 145.8825 88.205) (end 147.1425 86.945) (width 0.25) (layer "B.Cu") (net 8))
 (segment (start 130.385 88.205) (end 145.8825 88.205) (width 0.25) (layer "B.Cu") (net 8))
 (segment (start 121.4 79.22) (end 130.385 88.205) (width 0.25) (layer "B.Cu") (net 8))
 (segment (start 141.025 97.645) (end 148.025 104.645) (width 0.25) (layer "F.Cu") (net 3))
 (segment (start 143.7825 86.125) (end 144.6025 86.945) (width 0.25) (layer "F.Cu") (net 3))
 (segment (start 141.025 87.6375) (end 141.025 97.645) (width 0.25) (layer "F.Cu") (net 3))
 (segment (start 136.675 76.68) (end 140.3125 80.3175) (width 0.25) (layer "F.Cu") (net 3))
 (segment (start 140.3125 86.925) (end 141.025 87.6375) (width 0.25) (layer "F.Cu") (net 3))
 (segment (start 140.3125 80.3175) (end 140.3125 86.925) (width 0.25) (layer "F.Cu") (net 3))
 (segment (start 141.1125 86.125) (end 143.7825 86.125) (width 0.25) (layer "F.Cu") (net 3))
 (segment (start 140.3125 86.925) (end 141.1125 86.125) (width 0.25) (layer "F.Cu") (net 3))
 (segment (start 136.675 91.92) (end 146.86 102.105) (width 0.25) (layer "B.Cu") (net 13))
 (segment (start 146.86 102.105) (end 148.025 102.105) (width 0.25) (layer "B.Cu") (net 13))
 (segment (start 137.84 89.38) (end 136.675 89.38) (width 0.25) (layer "B.Cu") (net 14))
 (segment (start 148.025 99.565) (end 137.84 89.38) (width 0.25) (layer "B.Cu") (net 14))
 (segment (start 145.2 70.1) (end 145.275 70.025) (width 0.25) (layer "F.Cu") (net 4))
 (segment (start 145.675 69.625) (end 145.275 70.025) (width 0.25) (layer "F.Cu") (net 4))
 (segment (start 138.05 65.95) (end 144.35 65.95) (width 0.25) (layer "F.Cu") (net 4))
 (segment (start 145.275 70.025) (end 145.275 70.1) (width 0.25) (layer "F.Cu") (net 4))
 (segment (start 135.875 66) (end 138 66) (width 0.25) (layer "F.Cu") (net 4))
 (segment (start 144.35 65.95) (end 145.675 67.275) (width 0.25) (layer "F.Cu") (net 4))
 (segment (start 145.675 67.275) (end 145.675 69.625) (width 0.25) (layer "F.Cu") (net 4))
 (segment (start 145.275 70.1) (end 145.2 70.1) (width 0.25) (layer "F.Cu") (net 4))
 (segment (start 138 66) (end 138.05 65.95) (width 0.25) (layer "F.Cu") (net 4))
 (via (at 145.275 70.1) (size 0.8) (drill 0.4) (layers "F.Cu" "B.Cu") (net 4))
 (segment (start 145.275 81.1925) (end 144.6025 81.865) (width 0.25) (layer "B.Cu") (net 4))
 (segment (start 145.275 70.1) (end 145.275 81.1925) (width 0.25) (layer "B.Cu") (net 4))
 (segment (start 139.5 87.125) (end 136.675 84.3) (width 0.25) (layer "F.Cu") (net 5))
 (segment (start 140.2125 89.45) (end 139.5 88.7375) (width 0.25) (layer "F.Cu") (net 5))
 (segment (start 139.5 88.7375) (end 139.5 87.125) (width 0.25) (layer "F.Cu") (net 5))
 (segment (start 145.95 83.0575) (end 147.1425 81.865) (width 0.25) (layer "B.Cu") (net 5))
 (segment (start 145.089201 85.58) (end 145.95 84.719201) (width 0.25) (layer "B.Cu") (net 5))
 (segment (start 137.955 85.58) (end 145.089201 85.58) (width 0.25) (layer "B.Cu") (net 5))
 (segment (start 145.95 84.719201) (end 145.95 83.0575) (width 0.25) (layer "B.Cu") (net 5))
 (segment (start 136.675 84.3) (end 137.955 85.58) (width 0.25) (layer "B.Cu") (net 5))
 (segment (start 143.3225 83.125) (end 138.04 83.125) (width 0.25) (layer "B.Cu") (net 6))
 (segment (start 144.6025 84.405) (end 143.3225 83.125) (width 0.25) (layer "B.Cu") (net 6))
 (segment (start 138.04 83.125) (end 136.675 81.76) (width 0.25) (layer "B.Cu") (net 6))
 (segment (start 145.963528 83.226028) (end 147.1425 84.405) (width 0.25) (layer "F.Cu") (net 7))
 (segment (start 143.775 72.95) (end 143.775 79.024327) (width 0.25) (layer "F.Cu") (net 7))
 (segment (start 143.775 79.024327) (end 145.963528 81.212855) (width 0.25) (layer "F.Cu") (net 7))
 (segment (start 145.963528 81.212855) (end 145.963528 83.226028) (width 0.25) (layer "F.Cu") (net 7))
 (segment (start 135.2 68.975) (end 141.7 68.975) (width 0.25) (layer "F.Cu") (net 80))
 (segment (start 141.7 68.975) (end 143.775 71.05) (width 0.25) (layer "F.Cu") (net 80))
 (segment (start 134.05 66) (end 136.3 68.25) (width 0.25) (layer "F.Cu") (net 27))
 (segment (start 132.3625 66) (end 134.05 66) (width 0.25) (layer "F.Cu") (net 27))
 (segment (start 136.3 68.25) (end 144.35 68.25) (width 0.25) (layer "F.Cu") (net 27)))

